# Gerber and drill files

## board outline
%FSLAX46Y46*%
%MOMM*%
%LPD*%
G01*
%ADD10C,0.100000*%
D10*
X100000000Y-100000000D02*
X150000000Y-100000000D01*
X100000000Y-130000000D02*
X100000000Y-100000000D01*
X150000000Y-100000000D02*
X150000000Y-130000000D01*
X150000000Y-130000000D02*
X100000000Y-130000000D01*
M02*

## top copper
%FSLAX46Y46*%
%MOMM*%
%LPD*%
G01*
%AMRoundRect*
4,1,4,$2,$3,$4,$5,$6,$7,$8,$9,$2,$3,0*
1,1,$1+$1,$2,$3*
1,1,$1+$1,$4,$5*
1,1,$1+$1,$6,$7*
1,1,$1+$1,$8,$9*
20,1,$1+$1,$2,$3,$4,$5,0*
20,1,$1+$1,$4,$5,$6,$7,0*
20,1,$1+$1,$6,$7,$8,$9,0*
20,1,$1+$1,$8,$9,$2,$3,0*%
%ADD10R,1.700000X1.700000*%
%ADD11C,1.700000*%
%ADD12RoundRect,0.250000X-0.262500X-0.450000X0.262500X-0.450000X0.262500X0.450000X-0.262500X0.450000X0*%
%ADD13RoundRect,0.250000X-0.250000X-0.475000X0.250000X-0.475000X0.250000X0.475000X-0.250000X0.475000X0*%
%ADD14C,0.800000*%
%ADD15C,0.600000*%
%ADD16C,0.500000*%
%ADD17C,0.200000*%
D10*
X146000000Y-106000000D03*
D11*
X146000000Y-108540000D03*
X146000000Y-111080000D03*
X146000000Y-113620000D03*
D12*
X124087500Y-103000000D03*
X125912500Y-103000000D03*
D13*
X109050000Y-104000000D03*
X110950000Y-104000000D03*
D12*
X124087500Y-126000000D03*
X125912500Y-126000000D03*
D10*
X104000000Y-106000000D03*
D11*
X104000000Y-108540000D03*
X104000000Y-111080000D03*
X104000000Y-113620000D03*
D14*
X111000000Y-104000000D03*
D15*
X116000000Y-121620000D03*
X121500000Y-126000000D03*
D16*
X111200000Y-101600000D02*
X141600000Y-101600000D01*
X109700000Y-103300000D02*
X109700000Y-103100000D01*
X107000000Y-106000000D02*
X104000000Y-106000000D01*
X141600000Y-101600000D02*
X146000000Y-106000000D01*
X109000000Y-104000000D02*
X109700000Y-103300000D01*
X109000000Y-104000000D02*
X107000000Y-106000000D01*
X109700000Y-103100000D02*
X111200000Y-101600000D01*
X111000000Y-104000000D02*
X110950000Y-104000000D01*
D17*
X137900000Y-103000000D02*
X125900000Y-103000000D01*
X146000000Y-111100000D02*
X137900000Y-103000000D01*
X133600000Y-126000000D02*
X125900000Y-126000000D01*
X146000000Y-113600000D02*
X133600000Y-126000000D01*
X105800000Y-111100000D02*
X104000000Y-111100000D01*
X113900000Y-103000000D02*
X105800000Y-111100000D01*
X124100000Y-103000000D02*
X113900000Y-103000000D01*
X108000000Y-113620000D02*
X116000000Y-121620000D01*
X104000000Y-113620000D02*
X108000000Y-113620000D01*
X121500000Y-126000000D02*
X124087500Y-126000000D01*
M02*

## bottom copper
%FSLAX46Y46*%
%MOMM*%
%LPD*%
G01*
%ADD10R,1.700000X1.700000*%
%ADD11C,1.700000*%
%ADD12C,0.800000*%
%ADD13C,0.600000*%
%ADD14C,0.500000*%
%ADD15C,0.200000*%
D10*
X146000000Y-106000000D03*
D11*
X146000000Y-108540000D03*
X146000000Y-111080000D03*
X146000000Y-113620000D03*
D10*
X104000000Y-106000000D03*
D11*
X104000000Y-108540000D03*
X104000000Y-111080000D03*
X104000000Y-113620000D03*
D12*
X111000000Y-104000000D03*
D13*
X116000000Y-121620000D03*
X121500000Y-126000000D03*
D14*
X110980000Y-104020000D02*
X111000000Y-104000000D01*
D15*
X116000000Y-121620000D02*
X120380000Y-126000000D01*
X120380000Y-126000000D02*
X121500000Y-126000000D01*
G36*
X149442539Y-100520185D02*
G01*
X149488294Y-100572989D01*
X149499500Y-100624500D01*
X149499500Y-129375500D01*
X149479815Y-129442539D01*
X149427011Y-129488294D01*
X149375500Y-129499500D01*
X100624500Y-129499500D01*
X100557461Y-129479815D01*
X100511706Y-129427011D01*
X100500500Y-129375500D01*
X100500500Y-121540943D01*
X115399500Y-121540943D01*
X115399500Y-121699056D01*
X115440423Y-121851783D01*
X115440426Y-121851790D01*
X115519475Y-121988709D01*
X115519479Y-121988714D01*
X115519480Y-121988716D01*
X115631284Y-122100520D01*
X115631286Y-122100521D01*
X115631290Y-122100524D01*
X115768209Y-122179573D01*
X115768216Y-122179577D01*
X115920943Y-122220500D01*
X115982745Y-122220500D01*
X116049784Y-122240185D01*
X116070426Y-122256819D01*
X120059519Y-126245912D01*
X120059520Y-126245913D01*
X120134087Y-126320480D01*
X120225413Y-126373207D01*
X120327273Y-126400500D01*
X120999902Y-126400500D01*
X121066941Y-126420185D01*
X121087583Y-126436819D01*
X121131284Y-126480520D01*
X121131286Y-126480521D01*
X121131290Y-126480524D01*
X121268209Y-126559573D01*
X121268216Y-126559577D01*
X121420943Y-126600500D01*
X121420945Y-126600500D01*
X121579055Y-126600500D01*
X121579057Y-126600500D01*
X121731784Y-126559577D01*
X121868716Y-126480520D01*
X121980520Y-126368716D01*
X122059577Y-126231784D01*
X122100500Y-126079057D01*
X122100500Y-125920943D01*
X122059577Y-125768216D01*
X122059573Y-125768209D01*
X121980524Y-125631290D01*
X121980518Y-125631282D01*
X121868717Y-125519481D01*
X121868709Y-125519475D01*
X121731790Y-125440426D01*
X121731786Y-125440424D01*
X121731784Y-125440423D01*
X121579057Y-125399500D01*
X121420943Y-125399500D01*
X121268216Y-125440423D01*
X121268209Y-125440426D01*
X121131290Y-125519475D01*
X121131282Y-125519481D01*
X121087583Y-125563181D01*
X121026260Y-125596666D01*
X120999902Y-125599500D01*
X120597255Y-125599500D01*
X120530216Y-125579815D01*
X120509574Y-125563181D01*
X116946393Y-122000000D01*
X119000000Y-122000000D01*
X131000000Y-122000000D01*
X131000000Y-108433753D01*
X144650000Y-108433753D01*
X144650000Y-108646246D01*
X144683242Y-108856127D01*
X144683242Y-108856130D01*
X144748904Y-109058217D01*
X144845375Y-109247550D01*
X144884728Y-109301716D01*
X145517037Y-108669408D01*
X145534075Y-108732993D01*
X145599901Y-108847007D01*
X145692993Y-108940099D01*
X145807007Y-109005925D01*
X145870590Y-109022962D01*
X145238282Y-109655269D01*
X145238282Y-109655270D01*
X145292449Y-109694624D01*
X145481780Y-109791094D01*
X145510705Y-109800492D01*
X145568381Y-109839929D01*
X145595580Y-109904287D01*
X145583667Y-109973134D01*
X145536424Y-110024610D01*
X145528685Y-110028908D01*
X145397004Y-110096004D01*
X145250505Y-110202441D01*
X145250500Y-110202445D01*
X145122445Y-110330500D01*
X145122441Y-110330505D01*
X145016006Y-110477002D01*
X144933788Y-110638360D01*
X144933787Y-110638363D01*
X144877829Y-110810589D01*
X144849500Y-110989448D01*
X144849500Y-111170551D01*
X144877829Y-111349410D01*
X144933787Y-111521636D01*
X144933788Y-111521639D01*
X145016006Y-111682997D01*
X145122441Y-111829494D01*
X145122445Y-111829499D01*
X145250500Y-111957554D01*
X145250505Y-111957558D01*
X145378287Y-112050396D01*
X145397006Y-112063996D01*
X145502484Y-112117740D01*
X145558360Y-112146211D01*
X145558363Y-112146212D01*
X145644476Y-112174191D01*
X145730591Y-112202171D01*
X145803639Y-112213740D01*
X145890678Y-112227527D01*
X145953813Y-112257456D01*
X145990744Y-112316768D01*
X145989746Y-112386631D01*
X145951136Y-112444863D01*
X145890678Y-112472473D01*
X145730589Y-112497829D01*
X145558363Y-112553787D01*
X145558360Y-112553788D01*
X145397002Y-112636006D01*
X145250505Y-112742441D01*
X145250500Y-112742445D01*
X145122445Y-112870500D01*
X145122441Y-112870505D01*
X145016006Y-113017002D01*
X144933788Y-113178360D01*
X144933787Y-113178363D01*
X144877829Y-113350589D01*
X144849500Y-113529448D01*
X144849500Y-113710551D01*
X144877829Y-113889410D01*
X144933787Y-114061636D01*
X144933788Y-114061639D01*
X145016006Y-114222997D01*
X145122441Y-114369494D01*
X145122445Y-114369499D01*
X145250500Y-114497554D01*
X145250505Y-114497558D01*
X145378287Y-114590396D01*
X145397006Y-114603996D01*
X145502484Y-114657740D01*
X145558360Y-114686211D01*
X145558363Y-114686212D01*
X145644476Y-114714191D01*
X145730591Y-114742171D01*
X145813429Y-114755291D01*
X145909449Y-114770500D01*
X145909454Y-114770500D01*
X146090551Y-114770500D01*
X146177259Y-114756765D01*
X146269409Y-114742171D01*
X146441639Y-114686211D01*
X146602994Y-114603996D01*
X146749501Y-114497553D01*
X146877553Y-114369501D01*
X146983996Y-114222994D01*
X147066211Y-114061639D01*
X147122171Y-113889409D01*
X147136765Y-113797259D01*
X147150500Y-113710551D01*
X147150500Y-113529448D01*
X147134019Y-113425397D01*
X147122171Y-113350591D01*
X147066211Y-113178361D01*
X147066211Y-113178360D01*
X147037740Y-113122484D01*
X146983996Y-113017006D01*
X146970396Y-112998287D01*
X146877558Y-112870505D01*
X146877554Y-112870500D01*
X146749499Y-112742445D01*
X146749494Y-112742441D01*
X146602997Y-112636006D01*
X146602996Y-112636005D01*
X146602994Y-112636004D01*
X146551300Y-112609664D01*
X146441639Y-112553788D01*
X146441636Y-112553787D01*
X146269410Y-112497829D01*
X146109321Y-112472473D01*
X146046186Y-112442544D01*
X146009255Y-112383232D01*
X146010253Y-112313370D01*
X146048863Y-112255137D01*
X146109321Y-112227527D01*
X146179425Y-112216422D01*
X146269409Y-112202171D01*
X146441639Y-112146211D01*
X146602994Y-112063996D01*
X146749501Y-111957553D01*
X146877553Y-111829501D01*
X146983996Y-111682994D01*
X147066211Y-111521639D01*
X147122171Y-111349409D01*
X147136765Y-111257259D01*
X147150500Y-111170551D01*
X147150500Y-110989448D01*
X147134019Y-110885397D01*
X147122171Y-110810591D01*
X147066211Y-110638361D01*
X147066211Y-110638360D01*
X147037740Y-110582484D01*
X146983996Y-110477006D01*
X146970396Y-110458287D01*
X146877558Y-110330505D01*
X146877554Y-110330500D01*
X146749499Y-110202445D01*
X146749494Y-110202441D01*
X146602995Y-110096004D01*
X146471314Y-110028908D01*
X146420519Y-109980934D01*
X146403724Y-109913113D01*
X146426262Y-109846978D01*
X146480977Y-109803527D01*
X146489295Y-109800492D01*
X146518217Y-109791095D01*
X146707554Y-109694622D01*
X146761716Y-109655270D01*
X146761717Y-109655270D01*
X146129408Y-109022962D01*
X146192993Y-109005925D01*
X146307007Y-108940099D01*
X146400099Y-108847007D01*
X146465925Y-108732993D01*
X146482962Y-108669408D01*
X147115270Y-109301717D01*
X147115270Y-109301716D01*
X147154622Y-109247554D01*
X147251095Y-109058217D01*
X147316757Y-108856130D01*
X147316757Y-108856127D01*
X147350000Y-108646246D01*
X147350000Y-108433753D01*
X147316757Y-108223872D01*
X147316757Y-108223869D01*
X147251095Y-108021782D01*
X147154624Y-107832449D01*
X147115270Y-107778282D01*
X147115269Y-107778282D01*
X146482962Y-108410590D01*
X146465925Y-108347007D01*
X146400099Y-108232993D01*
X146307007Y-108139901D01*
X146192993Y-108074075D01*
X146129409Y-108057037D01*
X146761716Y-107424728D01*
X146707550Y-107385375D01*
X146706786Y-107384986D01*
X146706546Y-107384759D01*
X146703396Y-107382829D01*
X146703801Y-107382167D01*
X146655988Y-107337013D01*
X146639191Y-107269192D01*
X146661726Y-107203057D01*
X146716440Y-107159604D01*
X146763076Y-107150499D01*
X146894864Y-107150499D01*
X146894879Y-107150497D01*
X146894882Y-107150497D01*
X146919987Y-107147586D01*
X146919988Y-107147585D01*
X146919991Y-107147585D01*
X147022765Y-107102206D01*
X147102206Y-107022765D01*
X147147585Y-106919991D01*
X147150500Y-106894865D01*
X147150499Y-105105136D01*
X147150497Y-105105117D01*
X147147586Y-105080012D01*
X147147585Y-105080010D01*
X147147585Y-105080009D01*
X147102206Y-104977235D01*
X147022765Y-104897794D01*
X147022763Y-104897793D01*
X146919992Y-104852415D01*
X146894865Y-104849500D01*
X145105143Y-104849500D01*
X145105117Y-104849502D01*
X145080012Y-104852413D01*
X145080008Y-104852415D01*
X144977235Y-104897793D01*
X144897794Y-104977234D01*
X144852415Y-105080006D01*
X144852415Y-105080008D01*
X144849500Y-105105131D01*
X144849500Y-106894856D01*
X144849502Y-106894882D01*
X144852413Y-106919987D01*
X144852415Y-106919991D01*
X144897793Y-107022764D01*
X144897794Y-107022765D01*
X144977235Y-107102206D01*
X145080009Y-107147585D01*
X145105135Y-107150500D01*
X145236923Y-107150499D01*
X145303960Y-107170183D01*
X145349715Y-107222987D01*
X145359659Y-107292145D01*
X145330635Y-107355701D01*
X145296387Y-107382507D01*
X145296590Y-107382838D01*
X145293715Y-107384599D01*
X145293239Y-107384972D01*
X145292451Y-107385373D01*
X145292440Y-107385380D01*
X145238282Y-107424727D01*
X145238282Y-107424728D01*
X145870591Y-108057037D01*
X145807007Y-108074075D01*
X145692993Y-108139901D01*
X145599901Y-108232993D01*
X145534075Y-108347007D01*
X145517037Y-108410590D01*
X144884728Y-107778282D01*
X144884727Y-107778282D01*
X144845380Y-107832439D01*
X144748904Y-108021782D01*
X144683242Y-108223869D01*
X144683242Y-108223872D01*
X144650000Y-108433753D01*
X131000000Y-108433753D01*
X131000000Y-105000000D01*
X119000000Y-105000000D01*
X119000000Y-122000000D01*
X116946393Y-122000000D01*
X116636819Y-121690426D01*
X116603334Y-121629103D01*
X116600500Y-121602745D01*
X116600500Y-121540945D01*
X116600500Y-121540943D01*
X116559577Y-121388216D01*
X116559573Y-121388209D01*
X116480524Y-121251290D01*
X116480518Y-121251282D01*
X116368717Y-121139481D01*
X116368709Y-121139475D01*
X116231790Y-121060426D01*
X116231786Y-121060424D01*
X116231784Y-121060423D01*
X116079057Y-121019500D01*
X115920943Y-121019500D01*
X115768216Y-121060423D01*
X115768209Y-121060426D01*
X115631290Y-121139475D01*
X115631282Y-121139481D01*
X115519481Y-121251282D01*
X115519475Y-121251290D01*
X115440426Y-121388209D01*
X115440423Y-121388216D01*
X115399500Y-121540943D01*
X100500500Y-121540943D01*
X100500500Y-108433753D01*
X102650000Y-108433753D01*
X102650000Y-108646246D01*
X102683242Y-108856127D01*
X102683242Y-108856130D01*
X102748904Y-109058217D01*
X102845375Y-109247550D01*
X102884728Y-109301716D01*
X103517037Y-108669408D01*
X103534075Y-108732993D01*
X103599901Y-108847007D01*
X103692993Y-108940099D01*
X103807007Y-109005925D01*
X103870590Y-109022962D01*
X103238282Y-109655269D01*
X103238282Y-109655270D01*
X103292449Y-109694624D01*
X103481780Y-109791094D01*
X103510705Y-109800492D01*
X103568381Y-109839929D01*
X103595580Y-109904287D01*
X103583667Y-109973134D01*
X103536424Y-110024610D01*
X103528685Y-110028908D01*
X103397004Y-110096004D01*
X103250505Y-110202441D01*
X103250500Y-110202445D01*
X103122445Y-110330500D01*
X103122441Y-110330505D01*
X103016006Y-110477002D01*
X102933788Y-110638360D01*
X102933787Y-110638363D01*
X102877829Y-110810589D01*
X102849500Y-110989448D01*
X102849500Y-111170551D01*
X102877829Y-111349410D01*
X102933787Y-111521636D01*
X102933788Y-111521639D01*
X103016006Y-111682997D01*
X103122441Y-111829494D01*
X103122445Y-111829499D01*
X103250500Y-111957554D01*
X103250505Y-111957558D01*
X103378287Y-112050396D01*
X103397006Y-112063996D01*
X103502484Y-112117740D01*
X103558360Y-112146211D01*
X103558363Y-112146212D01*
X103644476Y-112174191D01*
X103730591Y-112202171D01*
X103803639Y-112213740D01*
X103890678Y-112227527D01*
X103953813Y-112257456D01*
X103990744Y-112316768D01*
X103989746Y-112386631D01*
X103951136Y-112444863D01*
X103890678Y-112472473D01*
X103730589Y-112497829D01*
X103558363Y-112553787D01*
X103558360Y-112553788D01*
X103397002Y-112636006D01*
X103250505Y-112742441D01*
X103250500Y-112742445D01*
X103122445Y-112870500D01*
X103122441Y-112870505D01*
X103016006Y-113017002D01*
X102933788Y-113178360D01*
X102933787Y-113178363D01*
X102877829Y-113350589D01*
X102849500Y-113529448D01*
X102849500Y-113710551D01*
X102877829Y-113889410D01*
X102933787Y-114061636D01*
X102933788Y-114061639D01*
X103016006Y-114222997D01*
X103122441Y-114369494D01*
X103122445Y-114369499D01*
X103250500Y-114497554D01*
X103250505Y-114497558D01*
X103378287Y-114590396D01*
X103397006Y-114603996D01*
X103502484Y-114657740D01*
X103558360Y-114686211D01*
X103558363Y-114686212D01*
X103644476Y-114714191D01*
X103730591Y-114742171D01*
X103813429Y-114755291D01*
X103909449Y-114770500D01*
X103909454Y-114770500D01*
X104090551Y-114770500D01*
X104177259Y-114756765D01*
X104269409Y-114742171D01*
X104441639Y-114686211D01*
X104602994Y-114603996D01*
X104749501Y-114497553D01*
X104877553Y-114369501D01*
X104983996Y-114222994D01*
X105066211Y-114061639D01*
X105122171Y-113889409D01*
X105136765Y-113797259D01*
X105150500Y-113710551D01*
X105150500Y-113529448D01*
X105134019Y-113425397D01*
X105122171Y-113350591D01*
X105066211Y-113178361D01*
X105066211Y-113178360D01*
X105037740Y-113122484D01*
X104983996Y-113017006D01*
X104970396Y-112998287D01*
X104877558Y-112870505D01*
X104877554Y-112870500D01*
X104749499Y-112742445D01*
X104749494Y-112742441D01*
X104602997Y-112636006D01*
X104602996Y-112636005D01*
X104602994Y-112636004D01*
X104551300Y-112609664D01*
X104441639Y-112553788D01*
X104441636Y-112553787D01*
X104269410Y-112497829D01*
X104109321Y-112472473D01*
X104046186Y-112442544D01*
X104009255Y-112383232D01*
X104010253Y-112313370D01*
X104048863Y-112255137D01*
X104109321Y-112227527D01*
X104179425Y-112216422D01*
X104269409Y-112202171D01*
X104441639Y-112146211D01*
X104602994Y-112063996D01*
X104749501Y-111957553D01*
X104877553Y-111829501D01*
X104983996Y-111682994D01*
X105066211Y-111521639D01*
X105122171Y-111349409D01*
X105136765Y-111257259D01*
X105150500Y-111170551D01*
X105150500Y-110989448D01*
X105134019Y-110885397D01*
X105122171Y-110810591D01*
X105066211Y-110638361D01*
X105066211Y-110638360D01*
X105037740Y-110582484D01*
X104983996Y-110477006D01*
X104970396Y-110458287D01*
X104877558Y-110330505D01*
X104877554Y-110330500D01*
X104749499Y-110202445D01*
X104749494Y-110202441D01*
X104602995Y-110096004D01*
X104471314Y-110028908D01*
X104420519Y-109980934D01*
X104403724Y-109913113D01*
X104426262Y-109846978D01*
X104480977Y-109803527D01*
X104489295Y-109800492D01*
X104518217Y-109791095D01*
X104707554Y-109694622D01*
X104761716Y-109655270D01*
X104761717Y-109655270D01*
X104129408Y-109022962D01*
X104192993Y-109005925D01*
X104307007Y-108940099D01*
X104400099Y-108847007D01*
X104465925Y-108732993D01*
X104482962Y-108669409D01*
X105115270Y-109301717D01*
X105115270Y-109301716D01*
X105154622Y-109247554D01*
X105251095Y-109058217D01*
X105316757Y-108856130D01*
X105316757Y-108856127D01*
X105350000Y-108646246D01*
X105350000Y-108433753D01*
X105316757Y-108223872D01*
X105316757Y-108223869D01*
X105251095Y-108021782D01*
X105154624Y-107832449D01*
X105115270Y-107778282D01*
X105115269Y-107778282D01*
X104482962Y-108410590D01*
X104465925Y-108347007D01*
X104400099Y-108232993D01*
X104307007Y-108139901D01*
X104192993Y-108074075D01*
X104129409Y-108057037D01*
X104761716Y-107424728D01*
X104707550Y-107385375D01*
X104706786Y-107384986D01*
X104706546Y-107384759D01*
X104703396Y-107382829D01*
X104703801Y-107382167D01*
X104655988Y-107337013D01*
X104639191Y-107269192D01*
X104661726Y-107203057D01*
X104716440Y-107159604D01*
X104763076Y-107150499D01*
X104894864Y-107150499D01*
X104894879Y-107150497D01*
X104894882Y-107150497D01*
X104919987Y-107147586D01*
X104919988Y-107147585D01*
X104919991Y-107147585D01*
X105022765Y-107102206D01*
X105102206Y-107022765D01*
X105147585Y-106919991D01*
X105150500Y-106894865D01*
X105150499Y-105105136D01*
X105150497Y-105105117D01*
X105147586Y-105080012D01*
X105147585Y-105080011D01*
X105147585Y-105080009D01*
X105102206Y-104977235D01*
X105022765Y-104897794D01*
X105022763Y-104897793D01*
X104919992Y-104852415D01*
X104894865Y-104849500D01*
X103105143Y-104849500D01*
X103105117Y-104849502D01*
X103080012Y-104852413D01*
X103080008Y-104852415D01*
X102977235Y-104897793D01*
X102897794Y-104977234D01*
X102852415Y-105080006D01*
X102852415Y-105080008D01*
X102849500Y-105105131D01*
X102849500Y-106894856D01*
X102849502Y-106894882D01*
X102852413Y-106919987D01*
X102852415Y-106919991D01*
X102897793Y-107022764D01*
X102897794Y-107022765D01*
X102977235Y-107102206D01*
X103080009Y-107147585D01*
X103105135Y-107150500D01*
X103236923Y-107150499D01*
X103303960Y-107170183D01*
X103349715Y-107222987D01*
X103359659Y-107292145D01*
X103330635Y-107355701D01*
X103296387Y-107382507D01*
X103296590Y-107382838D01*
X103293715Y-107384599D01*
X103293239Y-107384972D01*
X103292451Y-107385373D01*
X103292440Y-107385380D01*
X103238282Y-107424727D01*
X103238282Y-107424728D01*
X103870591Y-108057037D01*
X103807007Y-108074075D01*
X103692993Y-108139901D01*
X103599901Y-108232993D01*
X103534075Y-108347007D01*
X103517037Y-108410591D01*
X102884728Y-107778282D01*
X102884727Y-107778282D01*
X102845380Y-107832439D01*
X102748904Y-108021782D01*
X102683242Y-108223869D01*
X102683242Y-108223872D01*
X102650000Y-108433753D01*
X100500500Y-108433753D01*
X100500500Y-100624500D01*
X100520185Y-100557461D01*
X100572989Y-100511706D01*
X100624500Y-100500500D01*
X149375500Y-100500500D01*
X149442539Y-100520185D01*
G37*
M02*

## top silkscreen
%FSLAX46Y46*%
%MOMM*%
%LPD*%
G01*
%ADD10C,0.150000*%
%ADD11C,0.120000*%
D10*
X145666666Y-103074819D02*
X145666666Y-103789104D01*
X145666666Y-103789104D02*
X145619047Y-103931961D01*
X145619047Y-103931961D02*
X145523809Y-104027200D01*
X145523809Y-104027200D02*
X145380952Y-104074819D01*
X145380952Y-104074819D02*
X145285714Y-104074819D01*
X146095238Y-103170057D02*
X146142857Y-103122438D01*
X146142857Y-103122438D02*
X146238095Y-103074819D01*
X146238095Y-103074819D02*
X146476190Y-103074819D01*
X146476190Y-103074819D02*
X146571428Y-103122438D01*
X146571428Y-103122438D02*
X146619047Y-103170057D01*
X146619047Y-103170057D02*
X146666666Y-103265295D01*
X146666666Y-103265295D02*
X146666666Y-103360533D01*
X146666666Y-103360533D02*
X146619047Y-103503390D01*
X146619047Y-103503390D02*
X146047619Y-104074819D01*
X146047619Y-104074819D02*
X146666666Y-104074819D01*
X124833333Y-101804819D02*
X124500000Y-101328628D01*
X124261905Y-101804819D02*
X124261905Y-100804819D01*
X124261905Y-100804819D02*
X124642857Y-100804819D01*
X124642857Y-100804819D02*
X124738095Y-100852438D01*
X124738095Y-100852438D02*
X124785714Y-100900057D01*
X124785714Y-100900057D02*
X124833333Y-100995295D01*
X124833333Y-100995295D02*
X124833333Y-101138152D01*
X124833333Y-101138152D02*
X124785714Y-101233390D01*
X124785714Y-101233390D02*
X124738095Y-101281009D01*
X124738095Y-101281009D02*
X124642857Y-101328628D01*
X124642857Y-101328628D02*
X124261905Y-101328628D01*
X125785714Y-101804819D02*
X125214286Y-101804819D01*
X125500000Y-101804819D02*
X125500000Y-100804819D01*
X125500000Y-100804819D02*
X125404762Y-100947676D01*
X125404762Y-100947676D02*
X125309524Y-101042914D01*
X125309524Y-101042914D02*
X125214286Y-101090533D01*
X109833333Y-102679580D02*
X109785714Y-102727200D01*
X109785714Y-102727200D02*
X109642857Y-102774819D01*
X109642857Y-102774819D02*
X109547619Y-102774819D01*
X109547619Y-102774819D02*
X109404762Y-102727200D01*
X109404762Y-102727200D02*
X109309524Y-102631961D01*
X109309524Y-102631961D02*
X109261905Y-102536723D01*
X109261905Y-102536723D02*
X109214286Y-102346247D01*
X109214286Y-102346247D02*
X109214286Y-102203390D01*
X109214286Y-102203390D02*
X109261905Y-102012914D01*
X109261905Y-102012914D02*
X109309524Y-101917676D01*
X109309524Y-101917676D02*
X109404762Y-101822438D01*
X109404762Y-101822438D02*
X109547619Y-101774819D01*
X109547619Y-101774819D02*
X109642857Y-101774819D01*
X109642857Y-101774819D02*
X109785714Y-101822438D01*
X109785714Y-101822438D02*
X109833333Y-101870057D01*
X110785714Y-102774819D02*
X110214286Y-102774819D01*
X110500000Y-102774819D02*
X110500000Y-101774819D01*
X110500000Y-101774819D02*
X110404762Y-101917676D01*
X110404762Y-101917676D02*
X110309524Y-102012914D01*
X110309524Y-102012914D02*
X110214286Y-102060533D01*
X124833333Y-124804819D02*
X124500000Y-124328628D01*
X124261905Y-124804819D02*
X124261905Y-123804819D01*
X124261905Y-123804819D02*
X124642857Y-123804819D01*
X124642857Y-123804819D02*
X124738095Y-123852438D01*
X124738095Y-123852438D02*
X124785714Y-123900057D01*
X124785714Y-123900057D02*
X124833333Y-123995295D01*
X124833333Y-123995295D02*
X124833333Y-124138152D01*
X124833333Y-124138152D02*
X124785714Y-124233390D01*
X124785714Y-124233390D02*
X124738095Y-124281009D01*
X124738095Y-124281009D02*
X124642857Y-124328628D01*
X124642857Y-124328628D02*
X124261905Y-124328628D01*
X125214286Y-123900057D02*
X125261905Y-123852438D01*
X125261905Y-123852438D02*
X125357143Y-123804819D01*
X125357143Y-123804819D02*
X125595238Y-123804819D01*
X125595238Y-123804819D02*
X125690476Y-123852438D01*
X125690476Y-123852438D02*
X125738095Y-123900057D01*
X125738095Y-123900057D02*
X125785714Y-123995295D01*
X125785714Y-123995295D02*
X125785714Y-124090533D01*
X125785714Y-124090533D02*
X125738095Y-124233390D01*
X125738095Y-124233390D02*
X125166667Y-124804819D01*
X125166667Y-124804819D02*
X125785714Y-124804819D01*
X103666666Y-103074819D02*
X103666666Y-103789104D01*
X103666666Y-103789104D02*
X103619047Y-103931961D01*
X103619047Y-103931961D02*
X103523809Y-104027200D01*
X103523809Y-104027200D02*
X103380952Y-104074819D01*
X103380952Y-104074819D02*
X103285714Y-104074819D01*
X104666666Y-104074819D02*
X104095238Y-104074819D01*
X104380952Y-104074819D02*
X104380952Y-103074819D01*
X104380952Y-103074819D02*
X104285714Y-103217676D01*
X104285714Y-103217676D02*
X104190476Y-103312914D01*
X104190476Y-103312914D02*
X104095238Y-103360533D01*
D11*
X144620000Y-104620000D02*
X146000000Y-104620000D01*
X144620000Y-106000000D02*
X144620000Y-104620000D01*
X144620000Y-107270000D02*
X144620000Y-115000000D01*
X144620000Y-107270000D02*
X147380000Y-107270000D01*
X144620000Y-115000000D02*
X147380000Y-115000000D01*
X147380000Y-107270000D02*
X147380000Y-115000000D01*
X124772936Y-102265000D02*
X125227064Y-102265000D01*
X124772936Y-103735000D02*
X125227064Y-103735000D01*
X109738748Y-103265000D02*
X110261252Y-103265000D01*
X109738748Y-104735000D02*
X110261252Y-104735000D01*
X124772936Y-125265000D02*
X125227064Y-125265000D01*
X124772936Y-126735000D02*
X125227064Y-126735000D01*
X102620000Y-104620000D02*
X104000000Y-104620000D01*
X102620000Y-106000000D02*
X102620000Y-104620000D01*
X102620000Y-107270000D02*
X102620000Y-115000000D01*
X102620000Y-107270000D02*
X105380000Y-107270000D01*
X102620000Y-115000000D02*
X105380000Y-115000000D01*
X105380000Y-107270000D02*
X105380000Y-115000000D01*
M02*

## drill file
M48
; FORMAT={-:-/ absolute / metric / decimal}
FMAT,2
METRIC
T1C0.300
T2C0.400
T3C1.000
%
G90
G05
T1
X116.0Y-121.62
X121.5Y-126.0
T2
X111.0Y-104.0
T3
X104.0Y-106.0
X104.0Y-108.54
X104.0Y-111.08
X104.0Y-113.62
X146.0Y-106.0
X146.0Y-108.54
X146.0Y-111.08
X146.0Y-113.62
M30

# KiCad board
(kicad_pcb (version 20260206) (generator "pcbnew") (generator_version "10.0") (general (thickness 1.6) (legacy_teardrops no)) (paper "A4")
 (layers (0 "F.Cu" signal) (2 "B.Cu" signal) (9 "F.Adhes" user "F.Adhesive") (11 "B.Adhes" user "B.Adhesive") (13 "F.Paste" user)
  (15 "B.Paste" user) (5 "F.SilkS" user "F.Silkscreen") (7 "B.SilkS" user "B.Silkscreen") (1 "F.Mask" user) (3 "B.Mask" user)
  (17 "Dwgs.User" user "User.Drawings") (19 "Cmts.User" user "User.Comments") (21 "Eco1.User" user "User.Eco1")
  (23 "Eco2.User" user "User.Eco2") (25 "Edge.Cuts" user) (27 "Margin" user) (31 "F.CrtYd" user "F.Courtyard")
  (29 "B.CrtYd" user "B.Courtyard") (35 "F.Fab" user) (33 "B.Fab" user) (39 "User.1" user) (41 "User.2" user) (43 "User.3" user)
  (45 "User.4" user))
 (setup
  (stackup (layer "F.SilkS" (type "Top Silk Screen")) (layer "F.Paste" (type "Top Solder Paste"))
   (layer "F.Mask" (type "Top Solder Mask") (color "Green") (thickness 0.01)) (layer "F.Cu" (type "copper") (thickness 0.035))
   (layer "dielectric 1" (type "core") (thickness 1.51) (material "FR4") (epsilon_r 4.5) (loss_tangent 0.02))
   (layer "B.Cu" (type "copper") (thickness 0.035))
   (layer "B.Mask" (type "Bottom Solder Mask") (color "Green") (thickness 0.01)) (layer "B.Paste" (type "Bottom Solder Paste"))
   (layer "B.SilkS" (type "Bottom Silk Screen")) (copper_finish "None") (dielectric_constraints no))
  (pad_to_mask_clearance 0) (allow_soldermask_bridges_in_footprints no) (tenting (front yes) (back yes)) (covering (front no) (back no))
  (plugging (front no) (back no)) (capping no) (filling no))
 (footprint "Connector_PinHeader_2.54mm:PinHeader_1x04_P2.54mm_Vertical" (layer "F.Cu") (at 146 106)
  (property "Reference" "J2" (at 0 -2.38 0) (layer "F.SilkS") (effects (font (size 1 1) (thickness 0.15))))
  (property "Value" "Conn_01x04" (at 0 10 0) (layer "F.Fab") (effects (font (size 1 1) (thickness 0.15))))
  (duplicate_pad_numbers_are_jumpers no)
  (fp_line (start -1.38 -1.38) (end 0 -1.38) (stroke (width 0.12) (type solid)) (layer "F.SilkS"))
  (fp_line (start -1.38 0) (end -1.38 -1.38) (stroke (width 0.12) (type solid)) (layer "F.SilkS"))
  (fp_line (start -1.38 1.27) (end -1.38 9) (stroke (width 0.12) (type solid)) (layer "F.SilkS"))
  (fp_line (start -1.38 1.27) (end 1.38 1.27) (stroke (width 0.12) (type solid)) (layer "F.SilkS"))
  (fp_line (start -1.38 9) (end 1.38 9) (stroke (width 0.12) (type solid)) (layer "F.SilkS"))
  (fp_line (start 1.38 1.27) (end 1.38 9) (stroke (width 0.12) (type solid)) (layer "F.SilkS"))
  (pad "1" thru_hole rect (at 0 0) (size 1.7 1.7) (drill 1) (layers "*.Cu" "*.Mask") (remove_unused_layers no) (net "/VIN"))
  (pad "2" thru_hole circle (at 0 2.54) (size 1.7 1.7) (drill 1) (layers "*.Cu" "*.Mask") (remove_unused_layers no) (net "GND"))
  (pad "3" thru_hole circle (at 0 5.08) (size 1.7 1.7) (drill 1) (layers "*.Cu" "*.Mask") (remove_unused_layers no) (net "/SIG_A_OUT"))
  (pad "4" thru_hole circle (at 0 7.62) (size 1.7 1.7) (drill 1) (layers "*.Cu" "*.Mask") (remove_unused_layers no) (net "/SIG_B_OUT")))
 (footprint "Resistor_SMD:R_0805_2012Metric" (layer "F.Cu") (at 125 103)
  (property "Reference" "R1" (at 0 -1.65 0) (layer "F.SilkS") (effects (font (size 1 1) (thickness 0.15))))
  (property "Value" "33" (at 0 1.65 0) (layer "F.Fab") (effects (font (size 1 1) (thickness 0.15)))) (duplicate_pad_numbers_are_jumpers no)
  (fp_line (start -0.227064 -0.735) (end 0.227064 -0.735) (stroke (width 0.12) (type solid)) (layer "F.SilkS"))
  (fp_line (start -0.227064 0.735) (end 0.227064 0.735) (stroke (width 0.12) (type solid)) (layer "F.SilkS"))
  (pad "1" smd roundrect (at -0.9125 0) (size 1.025 1.4) (layers "F.Cu" "F.Mask" "F.Paste") (roundrect_rratio 0.243902) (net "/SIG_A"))
  (pad "2" smd roundrect (at 0.9125 0) (size 1.025 1.4) (layers "F.Cu" "F.Mask" "F.Paste") (roundrect_rratio 0.243902) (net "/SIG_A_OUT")))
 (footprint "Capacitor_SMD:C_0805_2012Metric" (layer "F.Cu") (at 110 104)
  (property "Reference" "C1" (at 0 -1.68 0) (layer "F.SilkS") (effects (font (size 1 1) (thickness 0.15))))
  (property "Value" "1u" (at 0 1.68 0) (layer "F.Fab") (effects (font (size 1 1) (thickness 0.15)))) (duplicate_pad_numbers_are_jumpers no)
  (fp_line (start -0.261252 -0.735) (end 0.261252 -0.735) (stroke (width 0.12) (type solid)) (layer "F.SilkS"))
  (fp_line (start -0.261252 0.735) (end 0.261252 0.735) (stroke (width 0.12) (type solid)) (layer "F.SilkS"))
  (pad "1" smd roundrect (at -0.95 0) (size 1 1.45) (layers "F.Cu" "F.Mask" "F.Paste") (roundrect_rratio 0.25) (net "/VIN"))
  (pad "2" smd roundrect (at 0.95 0) (size 1 1.45) (layers "F.Cu" "F.Mask" "F.Paste") (roundrect_rratio 0.25) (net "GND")))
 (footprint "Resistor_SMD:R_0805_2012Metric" (layer "F.Cu") (at 125 126)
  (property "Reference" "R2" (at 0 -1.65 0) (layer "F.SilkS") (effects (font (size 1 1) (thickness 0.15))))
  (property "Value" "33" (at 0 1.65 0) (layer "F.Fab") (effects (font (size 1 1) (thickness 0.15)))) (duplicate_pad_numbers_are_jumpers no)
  (fp_line (start -0.227064 -0.735) (end 0.227064 -0.735) (stroke (width 0.12) (type solid)) (layer "F.SilkS"))
  (fp_line (start -0.227064 0.735) (end 0.227064 0.735) (stroke (width 0.12) (type solid)) (layer "F.SilkS"))
  (pad "1" smd roundrect (at -0.9125 0) (size 1.025 1.4) (layers "F.Cu" "F.Mask" "F.Paste") (roundrect_rratio 0.243902) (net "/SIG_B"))
  (pad "2" smd roundrect (at 0.9125 0) (size 1.025 1.4) (layers "F.Cu" "F.Mask" "F.Paste") (roundrect_rratio 0.243902) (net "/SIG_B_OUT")))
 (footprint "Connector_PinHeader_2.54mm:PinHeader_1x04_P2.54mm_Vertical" (layer "F.Cu") (at 104 106)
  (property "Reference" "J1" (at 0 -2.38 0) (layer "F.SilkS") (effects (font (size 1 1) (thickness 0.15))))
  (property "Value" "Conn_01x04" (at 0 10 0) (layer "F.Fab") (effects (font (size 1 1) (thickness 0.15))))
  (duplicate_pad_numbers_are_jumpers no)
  (fp_line (start -1.38 -1.38) (end 0 -1.38) (stroke (width 0.12) (type solid)) (layer "F.SilkS"))
  (fp_line (start -1.38 0) (end -1.38 -1.38) (stroke (width 0.12) (type solid)) (layer "F.SilkS"))
  (fp_line (start -1.38 1.27) (end -1.38 9) (stroke (width 0.12) (type solid)) (layer "F.SilkS"))
  (fp_line (start -1.38 1.27) (end 1.38 1.27) (stroke (width 0.12) (type solid)) (layer "F.SilkS"))
  (fp_line (start -1.38 9) (end 1.38 9) (stroke (width 0.12) (type solid)) (layer "F.SilkS"))
  (fp_line (start 1.38 1.27) (end 1.38 9) (stroke (width 0.12) (type solid)) (layer "F.SilkS"))
  (pad "1" thru_hole rect (at 0 0) (size 1.7 1.7) (drill 1) (layers "*.Cu" "*.Mask") (remove_unused_layers no) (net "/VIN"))
  (pad "2" thru_hole circle (at 0 2.54) (size 1.7 1.7) (drill 1) (layers "*.Cu" "*.Mask") (remove_unused_layers no) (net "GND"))
  (pad "3" thru_hole circle (at 0 5.08) (size 1.7 1.7) (drill 1) (layers "*.Cu" "*.Mask") (remove_unused_layers no) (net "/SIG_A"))
  (pad "4" thru_hole circle (at 0 7.62) (size 1.7 1.7) (drill 1) (layers "*.Cu" "*.Mask") (remove_unused_layers no) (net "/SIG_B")))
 (gr_line (start 100 100) (end 150 100) (stroke (width 0.1) (type default)) (layer "Edge.Cuts"))
 (gr_line (start 100 130) (end 100 100) (stroke (width 0.1) (type default)) (layer "Edge.Cuts"))
 (gr_line (start 150 100) (end 150 130) (stroke (width 0.1) (type default)) (layer "Edge.Cuts"))
 (gr_line (start 150 130) (end 100 130) (stroke (width 0.1) (type default)) (layer "Edge.Cuts"))
 (segment (start 111.2 101.6) (end 141.6 101.6) (width 0.5) (layer "F.Cu") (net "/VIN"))
 (segment (start 109.7 103.3) (end 109.7 103.1) (width 0.5) (layer "F.Cu") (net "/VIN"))
 (segment (start 107 106) (end 104 106) (width 0.5) (layer "F.Cu") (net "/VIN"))
 (segment (start 141.6 101.6) (end 146 106) (width 0.5) (layer "F.Cu") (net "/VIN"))
 (segment (start 109 104) (end 109.7 103.3) (width 0.5) (layer "F.Cu") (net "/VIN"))
 (segment (start 109 104) (end 107 106) (width 0.5) (layer "F.Cu") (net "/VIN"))
 (segment (start 109.7 103.1) (end 111.2 101.6) (width 0.5) (layer "F.Cu") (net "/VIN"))
 (segment (start 111 104) (end 110.95 104) (width 0.5) (layer "F.Cu") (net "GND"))
 (via (at 111 104) (size 0.8) (drill 0.4) (layers "F.Cu" "B.Cu") (capping yes) (filling yes) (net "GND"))
 (segment (start 110.98 104.02) (end 111 104) (width 0.5) (layer "B.Cu") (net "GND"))
 (segment (start 137.9 103) (end 125.9 103) (width 0.2) (layer "F.Cu") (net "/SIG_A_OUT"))
 (segment (start 146 111.1) (end 137.9 103) (width 0.2) (layer "F.Cu") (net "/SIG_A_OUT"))
 (segment (start 133.6 126) (end 125.9 126) (width 0.2) (layer "F.Cu") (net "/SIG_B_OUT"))
 (segment (start 146 113.6) (end 133.6 126) (width 0.2) (layer "F.Cu") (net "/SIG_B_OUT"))
 (segment (start 105.8 111.1) (end 104 111.1) (width 0.2) (layer "F.Cu") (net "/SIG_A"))
 (segment (start 113.9 103) (end 105.8 111.1) (width 0.2) (layer "F.Cu") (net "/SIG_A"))
 (segment (start 124.1 103) (end 113.9 103) (width 0.2) (layer "F.Cu") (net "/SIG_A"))
 (segment (start 108 113.62) (end 116 121.62) (width 0.2) (locked yes) (layer "F.Cu") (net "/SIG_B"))
 (segment (start 104 113.62) (end 108 113.62) (width 0.2) (locked yes) (layer "F.Cu") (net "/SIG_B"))
 (segment (start 121.5 126) (end 124.0875 126) (width 0.2) (locked yes) (layer "F.Cu") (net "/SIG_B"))
 (via (at 116 121.62) (size 0.6) (drill 0.3) (layers "F.Cu" "B.Cu") (locked yes) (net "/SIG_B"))
 (via (at 121.5 126) (size 0.6) (drill 0.3) (layers "F.Cu" "B.Cu") (locked yes) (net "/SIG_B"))
 (segment (start 116 121.62) (end 120.38 126) (width 0.2) (locked yes) (layer "B.Cu") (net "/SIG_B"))
 (segment (start 120.38 126) (end 121.5 126) (width 0.2) (locked yes) (layer "B.Cu") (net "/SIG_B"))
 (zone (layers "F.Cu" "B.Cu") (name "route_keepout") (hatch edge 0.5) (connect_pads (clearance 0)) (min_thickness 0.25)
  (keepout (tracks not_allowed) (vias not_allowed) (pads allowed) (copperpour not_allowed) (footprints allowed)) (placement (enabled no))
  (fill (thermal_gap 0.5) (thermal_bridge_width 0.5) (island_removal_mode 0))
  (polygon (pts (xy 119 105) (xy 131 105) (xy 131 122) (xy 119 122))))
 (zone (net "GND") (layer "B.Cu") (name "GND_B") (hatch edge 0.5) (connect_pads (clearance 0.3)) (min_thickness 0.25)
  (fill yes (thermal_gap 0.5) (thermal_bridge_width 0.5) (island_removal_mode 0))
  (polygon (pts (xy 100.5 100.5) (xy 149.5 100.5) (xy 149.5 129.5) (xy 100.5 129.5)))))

